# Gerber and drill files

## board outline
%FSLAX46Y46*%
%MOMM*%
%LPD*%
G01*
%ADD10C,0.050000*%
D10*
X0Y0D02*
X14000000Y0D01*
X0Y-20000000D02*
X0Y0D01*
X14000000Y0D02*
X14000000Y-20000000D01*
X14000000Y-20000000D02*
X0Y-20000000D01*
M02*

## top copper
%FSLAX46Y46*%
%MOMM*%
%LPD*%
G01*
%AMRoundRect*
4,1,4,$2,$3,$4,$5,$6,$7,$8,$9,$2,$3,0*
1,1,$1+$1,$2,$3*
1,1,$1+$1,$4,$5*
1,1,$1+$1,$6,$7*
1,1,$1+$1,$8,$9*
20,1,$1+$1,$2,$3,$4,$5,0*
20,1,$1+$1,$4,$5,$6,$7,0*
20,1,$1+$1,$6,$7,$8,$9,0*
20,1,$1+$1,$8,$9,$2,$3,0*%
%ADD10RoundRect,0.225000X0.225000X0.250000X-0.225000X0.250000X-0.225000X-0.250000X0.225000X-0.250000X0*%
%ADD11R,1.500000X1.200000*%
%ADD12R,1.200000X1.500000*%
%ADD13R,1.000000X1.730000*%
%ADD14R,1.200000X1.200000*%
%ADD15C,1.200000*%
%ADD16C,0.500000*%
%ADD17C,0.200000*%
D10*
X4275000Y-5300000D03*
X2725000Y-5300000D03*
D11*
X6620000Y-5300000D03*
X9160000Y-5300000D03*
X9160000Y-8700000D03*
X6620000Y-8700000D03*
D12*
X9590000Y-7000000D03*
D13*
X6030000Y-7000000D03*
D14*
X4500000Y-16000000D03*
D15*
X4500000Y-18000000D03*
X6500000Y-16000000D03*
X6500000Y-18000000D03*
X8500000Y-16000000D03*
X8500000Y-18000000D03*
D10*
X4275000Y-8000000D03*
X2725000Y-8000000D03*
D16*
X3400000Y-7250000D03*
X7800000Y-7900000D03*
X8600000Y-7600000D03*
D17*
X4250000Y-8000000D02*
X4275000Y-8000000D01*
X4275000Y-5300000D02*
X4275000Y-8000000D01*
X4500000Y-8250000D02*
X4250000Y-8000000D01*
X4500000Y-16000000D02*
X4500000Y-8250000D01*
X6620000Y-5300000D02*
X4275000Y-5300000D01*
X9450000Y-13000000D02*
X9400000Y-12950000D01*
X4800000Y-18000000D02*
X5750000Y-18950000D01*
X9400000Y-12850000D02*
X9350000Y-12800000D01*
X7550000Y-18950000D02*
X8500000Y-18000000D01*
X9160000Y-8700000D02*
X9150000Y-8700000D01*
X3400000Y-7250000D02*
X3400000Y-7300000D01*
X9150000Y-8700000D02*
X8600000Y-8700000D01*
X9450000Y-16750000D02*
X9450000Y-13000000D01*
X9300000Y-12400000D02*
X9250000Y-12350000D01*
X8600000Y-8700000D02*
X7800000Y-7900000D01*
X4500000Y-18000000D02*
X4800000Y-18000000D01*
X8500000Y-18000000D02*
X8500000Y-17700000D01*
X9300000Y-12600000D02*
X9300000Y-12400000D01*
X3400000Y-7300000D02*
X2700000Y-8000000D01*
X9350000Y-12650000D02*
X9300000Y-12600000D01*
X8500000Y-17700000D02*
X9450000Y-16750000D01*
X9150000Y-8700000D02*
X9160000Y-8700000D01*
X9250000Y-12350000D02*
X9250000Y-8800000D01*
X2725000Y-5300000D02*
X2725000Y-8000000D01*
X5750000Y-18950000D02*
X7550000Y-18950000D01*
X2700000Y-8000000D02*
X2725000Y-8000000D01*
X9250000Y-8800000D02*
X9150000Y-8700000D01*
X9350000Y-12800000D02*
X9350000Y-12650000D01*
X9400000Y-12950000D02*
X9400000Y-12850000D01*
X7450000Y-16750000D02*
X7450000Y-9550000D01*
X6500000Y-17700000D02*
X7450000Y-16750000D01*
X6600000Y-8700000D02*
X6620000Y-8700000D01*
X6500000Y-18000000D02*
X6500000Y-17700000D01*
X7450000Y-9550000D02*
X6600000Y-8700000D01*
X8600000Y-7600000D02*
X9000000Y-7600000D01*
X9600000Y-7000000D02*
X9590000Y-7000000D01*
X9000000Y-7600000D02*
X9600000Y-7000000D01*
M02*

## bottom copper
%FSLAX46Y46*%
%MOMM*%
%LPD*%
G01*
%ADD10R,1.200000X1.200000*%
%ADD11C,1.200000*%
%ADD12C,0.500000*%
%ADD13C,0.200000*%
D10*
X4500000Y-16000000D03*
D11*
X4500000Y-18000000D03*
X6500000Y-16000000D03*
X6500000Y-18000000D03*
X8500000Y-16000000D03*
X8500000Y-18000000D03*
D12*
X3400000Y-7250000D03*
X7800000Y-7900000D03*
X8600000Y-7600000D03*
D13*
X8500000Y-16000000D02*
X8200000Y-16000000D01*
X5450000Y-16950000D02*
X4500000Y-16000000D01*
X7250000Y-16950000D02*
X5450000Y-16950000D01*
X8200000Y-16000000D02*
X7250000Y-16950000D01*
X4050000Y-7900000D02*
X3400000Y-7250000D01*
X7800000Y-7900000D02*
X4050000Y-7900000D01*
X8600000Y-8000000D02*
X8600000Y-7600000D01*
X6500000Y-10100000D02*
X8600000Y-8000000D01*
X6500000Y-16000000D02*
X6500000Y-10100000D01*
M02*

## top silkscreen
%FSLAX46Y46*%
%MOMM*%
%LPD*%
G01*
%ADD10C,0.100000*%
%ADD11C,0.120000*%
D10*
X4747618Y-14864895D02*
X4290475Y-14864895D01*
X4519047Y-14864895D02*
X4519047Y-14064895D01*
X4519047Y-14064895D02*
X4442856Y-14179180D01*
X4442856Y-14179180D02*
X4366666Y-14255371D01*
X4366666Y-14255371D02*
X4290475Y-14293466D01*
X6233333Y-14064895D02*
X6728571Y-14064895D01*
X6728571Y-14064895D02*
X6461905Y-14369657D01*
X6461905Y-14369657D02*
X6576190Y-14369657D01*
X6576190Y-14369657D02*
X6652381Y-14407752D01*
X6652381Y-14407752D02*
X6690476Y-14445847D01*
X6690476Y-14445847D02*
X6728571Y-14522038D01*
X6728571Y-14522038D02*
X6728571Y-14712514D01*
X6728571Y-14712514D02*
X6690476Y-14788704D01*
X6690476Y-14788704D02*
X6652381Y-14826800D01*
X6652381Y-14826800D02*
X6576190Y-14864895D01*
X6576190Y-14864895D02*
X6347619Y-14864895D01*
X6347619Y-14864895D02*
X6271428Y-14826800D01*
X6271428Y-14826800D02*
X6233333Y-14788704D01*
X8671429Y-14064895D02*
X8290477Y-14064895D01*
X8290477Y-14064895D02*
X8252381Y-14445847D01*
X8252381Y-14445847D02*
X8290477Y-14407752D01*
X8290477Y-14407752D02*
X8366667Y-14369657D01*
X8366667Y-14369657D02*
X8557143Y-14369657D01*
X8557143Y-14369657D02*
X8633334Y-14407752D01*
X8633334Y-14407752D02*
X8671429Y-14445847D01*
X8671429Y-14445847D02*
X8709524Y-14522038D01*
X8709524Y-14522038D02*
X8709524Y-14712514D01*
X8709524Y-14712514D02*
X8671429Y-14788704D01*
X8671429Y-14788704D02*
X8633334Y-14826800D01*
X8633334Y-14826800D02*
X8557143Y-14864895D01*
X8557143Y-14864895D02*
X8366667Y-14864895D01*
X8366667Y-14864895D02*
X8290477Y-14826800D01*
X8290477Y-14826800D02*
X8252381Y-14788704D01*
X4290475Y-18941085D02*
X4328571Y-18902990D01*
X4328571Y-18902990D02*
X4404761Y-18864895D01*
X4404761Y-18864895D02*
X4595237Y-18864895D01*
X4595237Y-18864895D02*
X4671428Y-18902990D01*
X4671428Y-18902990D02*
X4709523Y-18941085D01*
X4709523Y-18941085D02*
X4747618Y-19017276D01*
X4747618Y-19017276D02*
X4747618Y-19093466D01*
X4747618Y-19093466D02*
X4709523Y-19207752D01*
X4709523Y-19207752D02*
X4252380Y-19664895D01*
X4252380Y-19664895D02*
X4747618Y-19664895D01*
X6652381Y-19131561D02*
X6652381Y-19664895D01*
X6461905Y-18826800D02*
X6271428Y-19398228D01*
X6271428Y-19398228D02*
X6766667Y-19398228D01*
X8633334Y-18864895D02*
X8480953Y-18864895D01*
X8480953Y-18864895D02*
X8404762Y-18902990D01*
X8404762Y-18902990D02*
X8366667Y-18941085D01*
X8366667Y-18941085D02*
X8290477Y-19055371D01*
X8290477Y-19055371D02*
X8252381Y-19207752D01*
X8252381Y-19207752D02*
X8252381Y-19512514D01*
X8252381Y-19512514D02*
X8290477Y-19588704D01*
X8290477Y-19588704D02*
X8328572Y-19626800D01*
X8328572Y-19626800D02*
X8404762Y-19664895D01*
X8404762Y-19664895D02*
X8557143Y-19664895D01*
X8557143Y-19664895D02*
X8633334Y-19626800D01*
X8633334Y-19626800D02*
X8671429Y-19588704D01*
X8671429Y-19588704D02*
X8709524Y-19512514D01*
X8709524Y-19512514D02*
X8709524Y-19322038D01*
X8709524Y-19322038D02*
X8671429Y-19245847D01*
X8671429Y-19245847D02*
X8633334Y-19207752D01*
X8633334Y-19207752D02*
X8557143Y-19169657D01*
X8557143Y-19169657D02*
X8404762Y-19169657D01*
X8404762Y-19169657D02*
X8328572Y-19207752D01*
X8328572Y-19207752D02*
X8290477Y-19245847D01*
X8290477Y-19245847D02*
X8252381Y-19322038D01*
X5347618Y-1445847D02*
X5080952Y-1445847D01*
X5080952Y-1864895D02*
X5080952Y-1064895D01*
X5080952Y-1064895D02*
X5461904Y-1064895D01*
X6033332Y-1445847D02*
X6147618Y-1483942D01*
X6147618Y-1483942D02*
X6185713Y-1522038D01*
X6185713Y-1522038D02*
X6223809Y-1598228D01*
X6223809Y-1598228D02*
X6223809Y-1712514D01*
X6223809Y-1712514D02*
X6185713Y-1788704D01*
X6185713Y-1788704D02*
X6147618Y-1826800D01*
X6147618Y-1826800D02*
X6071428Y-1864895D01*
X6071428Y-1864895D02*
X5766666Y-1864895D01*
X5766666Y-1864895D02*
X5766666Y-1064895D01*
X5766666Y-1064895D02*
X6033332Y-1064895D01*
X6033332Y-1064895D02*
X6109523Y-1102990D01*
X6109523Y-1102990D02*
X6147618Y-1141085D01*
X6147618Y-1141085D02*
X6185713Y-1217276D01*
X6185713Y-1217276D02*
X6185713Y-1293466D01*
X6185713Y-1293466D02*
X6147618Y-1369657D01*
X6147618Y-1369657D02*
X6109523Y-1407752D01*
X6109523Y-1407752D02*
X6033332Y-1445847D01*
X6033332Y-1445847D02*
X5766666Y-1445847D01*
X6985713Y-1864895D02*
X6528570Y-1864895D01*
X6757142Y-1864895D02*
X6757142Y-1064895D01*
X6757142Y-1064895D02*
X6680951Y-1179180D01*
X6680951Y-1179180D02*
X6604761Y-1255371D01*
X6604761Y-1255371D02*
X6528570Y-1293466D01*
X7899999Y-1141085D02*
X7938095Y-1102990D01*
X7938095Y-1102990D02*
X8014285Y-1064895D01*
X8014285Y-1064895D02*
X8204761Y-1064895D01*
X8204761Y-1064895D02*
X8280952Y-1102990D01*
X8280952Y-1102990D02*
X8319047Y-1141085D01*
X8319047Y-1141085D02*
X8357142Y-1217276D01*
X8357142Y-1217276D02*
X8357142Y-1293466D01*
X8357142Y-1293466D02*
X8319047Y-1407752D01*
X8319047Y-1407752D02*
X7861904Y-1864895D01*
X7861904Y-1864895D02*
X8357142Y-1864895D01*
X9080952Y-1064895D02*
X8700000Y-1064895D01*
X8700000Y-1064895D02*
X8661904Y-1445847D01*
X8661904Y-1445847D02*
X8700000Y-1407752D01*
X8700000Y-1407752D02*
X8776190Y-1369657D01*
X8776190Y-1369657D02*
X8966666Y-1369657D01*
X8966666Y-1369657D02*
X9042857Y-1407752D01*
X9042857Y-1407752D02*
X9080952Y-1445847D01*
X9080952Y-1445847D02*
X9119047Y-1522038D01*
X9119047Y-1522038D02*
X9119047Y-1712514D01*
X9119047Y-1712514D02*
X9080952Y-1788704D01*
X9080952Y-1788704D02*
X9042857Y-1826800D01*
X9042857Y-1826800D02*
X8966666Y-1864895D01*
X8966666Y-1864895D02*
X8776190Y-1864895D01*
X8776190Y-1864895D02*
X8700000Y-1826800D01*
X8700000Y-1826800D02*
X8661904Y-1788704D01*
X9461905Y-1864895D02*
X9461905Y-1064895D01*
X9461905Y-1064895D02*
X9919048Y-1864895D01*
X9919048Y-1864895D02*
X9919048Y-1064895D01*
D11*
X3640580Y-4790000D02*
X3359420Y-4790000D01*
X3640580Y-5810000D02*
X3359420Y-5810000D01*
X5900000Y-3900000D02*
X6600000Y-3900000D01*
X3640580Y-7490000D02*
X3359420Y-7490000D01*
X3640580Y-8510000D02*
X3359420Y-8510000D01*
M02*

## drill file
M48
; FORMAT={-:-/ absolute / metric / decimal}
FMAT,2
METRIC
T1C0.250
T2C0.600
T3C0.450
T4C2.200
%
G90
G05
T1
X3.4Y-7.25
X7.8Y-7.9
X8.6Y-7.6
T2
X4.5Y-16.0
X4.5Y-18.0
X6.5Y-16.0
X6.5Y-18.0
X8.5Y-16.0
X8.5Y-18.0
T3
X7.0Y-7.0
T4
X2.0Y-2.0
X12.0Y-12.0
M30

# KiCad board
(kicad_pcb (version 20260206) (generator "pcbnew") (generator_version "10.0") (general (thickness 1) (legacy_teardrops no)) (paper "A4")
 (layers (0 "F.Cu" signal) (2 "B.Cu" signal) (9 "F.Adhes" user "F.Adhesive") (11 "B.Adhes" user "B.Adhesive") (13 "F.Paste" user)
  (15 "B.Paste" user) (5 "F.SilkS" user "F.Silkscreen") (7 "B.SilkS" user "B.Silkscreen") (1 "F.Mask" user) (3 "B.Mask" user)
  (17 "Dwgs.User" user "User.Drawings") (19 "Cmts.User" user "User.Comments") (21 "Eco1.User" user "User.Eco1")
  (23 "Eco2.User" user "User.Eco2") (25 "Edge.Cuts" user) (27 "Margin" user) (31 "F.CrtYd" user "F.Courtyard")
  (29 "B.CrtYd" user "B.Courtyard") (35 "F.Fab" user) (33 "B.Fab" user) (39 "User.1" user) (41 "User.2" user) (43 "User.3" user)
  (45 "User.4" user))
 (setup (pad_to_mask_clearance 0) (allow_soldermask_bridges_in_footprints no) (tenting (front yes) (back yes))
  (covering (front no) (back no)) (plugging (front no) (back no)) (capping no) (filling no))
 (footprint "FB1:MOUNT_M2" (layer "F.Cu") (at 2 2)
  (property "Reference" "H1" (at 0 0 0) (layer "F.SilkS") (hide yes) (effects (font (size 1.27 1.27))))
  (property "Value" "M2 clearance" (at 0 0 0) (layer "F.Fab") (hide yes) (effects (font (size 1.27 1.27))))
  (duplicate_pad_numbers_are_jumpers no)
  (pad "" np_thru_hole circle (at 0 0) (size 2.2 2.2) (drill 2.2) (layers "*.Cu")))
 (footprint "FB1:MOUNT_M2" (layer "F.Cu") (at 12 12)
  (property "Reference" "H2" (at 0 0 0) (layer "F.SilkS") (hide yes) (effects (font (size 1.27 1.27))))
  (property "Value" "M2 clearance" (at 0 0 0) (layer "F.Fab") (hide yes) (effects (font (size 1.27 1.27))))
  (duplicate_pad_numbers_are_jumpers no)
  (pad "" np_thru_hole circle (at 0 0) (size 2.2 2.2) (drill 2.2) (layers "*.Cu")))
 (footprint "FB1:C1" (layer "F.Cu") (at 3.5 5.3 180)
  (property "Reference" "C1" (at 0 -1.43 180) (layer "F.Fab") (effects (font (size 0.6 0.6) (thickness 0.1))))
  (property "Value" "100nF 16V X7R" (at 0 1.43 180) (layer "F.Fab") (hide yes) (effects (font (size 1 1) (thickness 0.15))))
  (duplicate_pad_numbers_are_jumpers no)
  (fp_line (start -0.14058 0.51) (end 0.14058 0.51) (stroke (width 0.12) (type solid)) (layer "F.SilkS"))
  (fp_line (start -0.14058 -0.51) (end 0.14058 -0.51) (stroke (width 0.12) (type solid)) (layer "F.SilkS"))
  (pad "1" smd roundrect (at -0.775 0 180) (size 0.9 0.95) (layers "F.Cu" "F.Mask" "F.Paste") (roundrect_rratio 0.25) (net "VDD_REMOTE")
   (solder_mask_margin 0.025))
  (pad "2" smd roundrect (at 0.775 0 180) (size 0.9 0.95) (layers "F.Cu" "F.Mask" "F.Paste") (roundrect_rratio 0.25) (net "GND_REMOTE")
   (solder_mask_margin 0.025)))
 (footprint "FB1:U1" (layer "F.Cu") (at 7 7)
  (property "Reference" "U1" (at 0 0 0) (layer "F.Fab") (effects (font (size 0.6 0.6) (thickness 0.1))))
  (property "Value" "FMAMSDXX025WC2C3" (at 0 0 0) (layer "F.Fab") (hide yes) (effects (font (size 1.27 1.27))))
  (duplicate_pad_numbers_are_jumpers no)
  (fp_line (start -1.1 -3.1) (end -0.4 -3.1) (stroke (width 0.12) (type default)) (layer "F.SilkS"))
  (pad "" np_thru_hole circle (at 0 0) (size 0.45 0.45) (drill 0.45) (layers "*.Cu") (solder_mask_margin 0.025))
  (pad "1" smd rect (at -0.38 -1.7) (size 1.5 1.2) (layers "F.Cu" "F.Mask" "F.Paste") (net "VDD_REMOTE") (solder_mask_margin 0.025)
   (thermal_bridge_angle 45))
  (pad "2" smd rect (at 2.16 -1.7) (size 1.5 1.2) (layers "F.Cu" "F.Mask" "F.Paste") (solder_mask_margin 0.025) (thermal_bridge_angle 45))
  (pad "3" smd rect (at 2.16 1.7) (size 1.5 1.2) (layers "F.Cu" "F.Mask" "F.Paste") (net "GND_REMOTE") (solder_mask_margin 0.025)
   (thermal_bridge_angle 45))
  (pad "4" smd rect (at -0.38 1.7) (size 1.5 1.2) (layers "F.Cu" "F.Mask" "F.Paste") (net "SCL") (solder_mask_margin 0.025)
   (thermal_bridge_angle 45))
  (pad "5" smd rect (at 2.59 0) (size 1.2 1.5) (layers "F.Cu" "F.Mask" "F.Paste") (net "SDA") (solder_mask_margin 0.025)
   (thermal_bridge_angle 45))
  (pad "6" smd rect (at -0.97 0) (size 1 1.73) (layers "F.Cu" "F.Mask" "F.Paste") (solder_mask_margin 0.025) (thermal_bridge_angle 45)))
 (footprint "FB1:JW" (layer "F.Cu") (at 0 0)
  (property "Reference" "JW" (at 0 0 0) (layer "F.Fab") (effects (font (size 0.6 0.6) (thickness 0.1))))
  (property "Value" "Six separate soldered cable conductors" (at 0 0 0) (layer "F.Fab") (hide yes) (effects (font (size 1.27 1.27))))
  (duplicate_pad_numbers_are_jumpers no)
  (pad "1" thru_hole rect (at 4.5 16) (size 1.2 1.2) (drill 0.6) (layers "*.Cu") (remove_unused_layers no) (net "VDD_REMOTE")
   (solder_mask_margin 0.025) (thermal_bridge_angle 45))
  (pad "2" thru_hole circle (at 4.5 18) (size 1.2 1.2) (drill 0.6) (layers "*.Cu") (remove_unused_layers no) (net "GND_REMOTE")
   (solder_mask_margin 0.025))
  (pad "3" thru_hole circle (at 6.5 16) (size 1.2 1.2) (drill 0.6) (layers "*.Cu") (remove_unused_layers no) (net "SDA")
   (solder_mask_margin 0.025))
  (pad "4" thru_hole circle (at 6.5 18) (size 1.2 1.2) (drill 0.6) (layers "*.Cu") (remove_unused_layers no) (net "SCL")
   (solder_mask_margin 0.025))
  (pad "5" thru_hole circle (at 8.5 16) (size 1.2 1.2) (drill 0.6) (layers "*.Cu") (remove_unused_layers no) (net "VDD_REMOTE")
   (solder_mask_margin 0.025))
  (pad "6" thru_hole circle (at 8.5 18) (size 1.2 1.2) (drill 0.6) (layers "*.Cu") (remove_unused_layers no) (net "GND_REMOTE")
   (solder_mask_margin 0.025)))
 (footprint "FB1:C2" (layer "F.Cu") (at 3.5 8 180)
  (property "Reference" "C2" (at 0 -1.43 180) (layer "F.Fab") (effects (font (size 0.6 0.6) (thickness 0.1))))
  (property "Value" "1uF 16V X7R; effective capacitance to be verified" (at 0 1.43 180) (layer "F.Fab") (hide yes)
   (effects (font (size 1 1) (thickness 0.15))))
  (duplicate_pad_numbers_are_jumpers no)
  (fp_line (start -0.14058 0.51) (end 0.14058 0.51) (stroke (width 0.12) (type solid)) (layer "F.SilkS"))
  (fp_line (start -0.14058 -0.51) (end 0.14058 -0.51) (stroke (width 0.12) (type solid)) (layer "F.SilkS"))
  (pad "1" smd roundrect (at -0.775 0 180) (size 0.9 0.95) (layers "F.Cu" "F.Mask" "F.Paste") (roundrect_rratio 0.25) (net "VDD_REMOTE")
   (solder_mask_margin 0.025))
  (pad "2" smd roundrect (at 0.775 0 180) (size 0.9 0.95) (layers "F.Cu" "F.Mask" "F.Paste") (roundrect_rratio 0.25) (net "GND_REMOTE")
   (solder_mask_margin 0.025)))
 (gr_line (start 0 0) (end 14 0) (stroke (width 0.05) (type default)) (layer "Edge.Cuts"))
 (gr_line (start 0 20) (end 0 0) (stroke (width 0.05) (type default)) (layer "Edge.Cuts"))
 (gr_line (start 14 0) (end 14 20) (stroke (width 0.05) (type default)) (layer "Edge.Cuts"))
 (gr_line (start 14 20) (end 0 20) (stroke (width 0.05) (type default)) (layer "Edge.Cuts"))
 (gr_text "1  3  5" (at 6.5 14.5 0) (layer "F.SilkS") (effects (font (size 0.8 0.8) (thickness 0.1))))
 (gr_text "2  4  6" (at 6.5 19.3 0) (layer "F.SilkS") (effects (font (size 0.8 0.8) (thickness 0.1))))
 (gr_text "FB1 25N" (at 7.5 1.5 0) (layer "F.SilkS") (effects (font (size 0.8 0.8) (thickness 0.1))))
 (segment (start 4.25 8) (end 4.275 8) (width 0.2) (layer "F.Cu") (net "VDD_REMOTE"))
 (segment (start 4.275 5.3) (end 4.275 8) (width 0.2) (layer "F.Cu") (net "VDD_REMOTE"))
 (segment (start 4.5 8.25) (end 4.25 8) (width 0.2) (layer "F.Cu") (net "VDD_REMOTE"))
 (segment (start 4.5 16) (end 4.5 8.25) (width 0.2) (layer "F.Cu") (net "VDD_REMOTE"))
 (segment (start 6.62 5.3) (end 4.275 5.3) (width 0.2) (layer "F.Cu") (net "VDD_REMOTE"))
 (segment (start 8.5 16) (end 8.2 16) (width 0.2) (layer "B.Cu") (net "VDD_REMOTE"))
 (segment (start 5.45 16.95) (end 4.5 16) (width 0.2) (layer "B.Cu") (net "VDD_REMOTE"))
 (segment (start 7.25 16.95) (end 5.45 16.95) (width 0.2) (layer "B.Cu") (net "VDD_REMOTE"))
 (segment (start 8.2 16) (end 7.25 16.95) (width 0.2) (layer "B.Cu") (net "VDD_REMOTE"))
 (segment (start 9.45 13) (end 9.4 12.95) (width 0.2) (layer "F.Cu") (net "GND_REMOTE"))
 (segment (start 4.8 18) (end 5.75 18.95) (width 0.2) (layer "F.Cu") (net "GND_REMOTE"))
 (segment (start 9.4 12.85) (end 9.35 12.8) (width 0.2) (layer "F.Cu") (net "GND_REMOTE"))
 (segment (start 7.55 18.95) (end 8.5 18) (width 0.2) (layer "F.Cu") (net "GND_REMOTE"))
 (segment (start 9.16 8.7) (end 9.15 8.7) (width 0.2) (layer "F.Cu") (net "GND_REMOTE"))
 (segment (start 3.4 7.25) (end 3.4 7.3) (width 0.2) (layer "F.Cu") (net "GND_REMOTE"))
 (segment (start 9.15 8.7) (end 8.6 8.7) (width 0.2) (layer "F.Cu") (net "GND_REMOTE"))
 (segment (start 9.45 16.75) (end 9.45 13) (width 0.2) (layer "F.Cu") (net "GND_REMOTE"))
 (segment (start 9.3 12.4) (end 9.25 12.35) (width 0.2) (layer "F.Cu") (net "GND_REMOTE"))
 (segment (start 8.6 8.7) (end 7.8 7.9) (width 0.2) (layer "F.Cu") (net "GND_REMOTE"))
 (segment (start 4.5 18) (end 4.8 18) (width 0.2) (layer "F.Cu") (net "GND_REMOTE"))
 (segment (start 8.5 18) (end 8.5 17.7) (width 0.2) (layer "F.Cu") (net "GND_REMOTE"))
 (segment (start 9.3 12.6) (end 9.3 12.4) (width 0.2) (layer "F.Cu") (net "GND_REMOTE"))
 (segment (start 3.4 7.3) (end 2.7 8) (width 0.2) (layer "F.Cu") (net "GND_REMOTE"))
 (segment (start 9.35 12.65) (end 9.3 12.6) (width 0.2) (layer "F.Cu") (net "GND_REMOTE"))
 (segment (start 8.5 17.7) (end 9.45 16.75) (width 0.2) (layer "F.Cu") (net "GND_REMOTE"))
 (segment (start 9.15 8.7) (end 9.16 8.7) (width 0.2) (layer "F.Cu") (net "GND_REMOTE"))
 (segment (start 9.25 12.35) (end 9.25 8.8) (width 0.2) (layer "F.Cu") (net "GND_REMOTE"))
 (segment (start 2.725 5.3) (end 2.725 8) (width 0.2) (layer "F.Cu") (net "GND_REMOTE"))
 (segment (start 5.75 18.95) (end 7.55 18.95) (width 0.2) (layer "F.Cu") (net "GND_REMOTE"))
 (segment (start 2.7 8) (end 2.725 8) (width 0.2) (layer "F.Cu") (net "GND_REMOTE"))
 (segment (start 9.25 8.8) (end 9.15 8.7) (width 0.2) (layer "F.Cu") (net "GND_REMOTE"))
 (segment (start 9.35 12.8) (end 9.35 12.65) (width 0.2) (layer "F.Cu") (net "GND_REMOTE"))
 (segment (start 9.4 12.95) (end 9.4 12.85) (width 0.2) (layer "F.Cu") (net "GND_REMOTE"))
 (via (at 3.4 7.25) (size 0.5) (drill 0.25) (layers "F.Cu" "B.Cu") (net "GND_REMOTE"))
 (via (at 7.8 7.9) (size 0.5) (drill 0.25) (layers "F.Cu" "B.Cu") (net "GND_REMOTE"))
 (segment (start 4.05 7.9) (end 3.4 7.25) (width 0.2) (layer "B.Cu") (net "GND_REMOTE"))
 (segment (start 7.8 7.9) (end 4.05 7.9) (width 0.2) (layer "B.Cu") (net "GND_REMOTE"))
 (segment (start 7.45 16.75) (end 7.45 9.55) (width 0.2) (layer "F.Cu") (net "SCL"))
 (segment (start 6.5 17.7) (end 7.45 16.75) (width 0.2) (layer "F.Cu") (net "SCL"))
 (segment (start 6.6 8.7) (end 6.62 8.7) (width 0.2) (layer "F.Cu") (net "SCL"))
 (segment (start 6.5 18) (end 6.5 17.7) (width 0.2) (layer "F.Cu") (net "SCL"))
 (segment (start 7.45 9.55) (end 6.6 8.7) (width 0.2) (layer "F.Cu") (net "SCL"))
 (segment (start 8.6 7.6) (end 9 7.6) (width 0.2) (layer "F.Cu") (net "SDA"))
 (segment (start 9.6 7) (end 9.59 7) (width 0.2) (layer "F.Cu") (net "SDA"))
 (segment (start 9 7.6) (end 9.6 7) (width 0.2) (layer "F.Cu") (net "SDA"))
 (via (at 8.6 7.6) (size 0.5) (drill 0.25) (layers "F.Cu" "B.Cu") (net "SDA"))
 (segment (start 8.6 8) (end 8.6 7.6) (width 0.2) (layer "B.Cu") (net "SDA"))
 (segment (start 6.5 10.1) (end 8.6 8) (width 0.2) (layer "B.Cu") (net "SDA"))
 (segment (start 6.5 16) (end 6.5 10.1) (width 0.2) (layer "B.Cu") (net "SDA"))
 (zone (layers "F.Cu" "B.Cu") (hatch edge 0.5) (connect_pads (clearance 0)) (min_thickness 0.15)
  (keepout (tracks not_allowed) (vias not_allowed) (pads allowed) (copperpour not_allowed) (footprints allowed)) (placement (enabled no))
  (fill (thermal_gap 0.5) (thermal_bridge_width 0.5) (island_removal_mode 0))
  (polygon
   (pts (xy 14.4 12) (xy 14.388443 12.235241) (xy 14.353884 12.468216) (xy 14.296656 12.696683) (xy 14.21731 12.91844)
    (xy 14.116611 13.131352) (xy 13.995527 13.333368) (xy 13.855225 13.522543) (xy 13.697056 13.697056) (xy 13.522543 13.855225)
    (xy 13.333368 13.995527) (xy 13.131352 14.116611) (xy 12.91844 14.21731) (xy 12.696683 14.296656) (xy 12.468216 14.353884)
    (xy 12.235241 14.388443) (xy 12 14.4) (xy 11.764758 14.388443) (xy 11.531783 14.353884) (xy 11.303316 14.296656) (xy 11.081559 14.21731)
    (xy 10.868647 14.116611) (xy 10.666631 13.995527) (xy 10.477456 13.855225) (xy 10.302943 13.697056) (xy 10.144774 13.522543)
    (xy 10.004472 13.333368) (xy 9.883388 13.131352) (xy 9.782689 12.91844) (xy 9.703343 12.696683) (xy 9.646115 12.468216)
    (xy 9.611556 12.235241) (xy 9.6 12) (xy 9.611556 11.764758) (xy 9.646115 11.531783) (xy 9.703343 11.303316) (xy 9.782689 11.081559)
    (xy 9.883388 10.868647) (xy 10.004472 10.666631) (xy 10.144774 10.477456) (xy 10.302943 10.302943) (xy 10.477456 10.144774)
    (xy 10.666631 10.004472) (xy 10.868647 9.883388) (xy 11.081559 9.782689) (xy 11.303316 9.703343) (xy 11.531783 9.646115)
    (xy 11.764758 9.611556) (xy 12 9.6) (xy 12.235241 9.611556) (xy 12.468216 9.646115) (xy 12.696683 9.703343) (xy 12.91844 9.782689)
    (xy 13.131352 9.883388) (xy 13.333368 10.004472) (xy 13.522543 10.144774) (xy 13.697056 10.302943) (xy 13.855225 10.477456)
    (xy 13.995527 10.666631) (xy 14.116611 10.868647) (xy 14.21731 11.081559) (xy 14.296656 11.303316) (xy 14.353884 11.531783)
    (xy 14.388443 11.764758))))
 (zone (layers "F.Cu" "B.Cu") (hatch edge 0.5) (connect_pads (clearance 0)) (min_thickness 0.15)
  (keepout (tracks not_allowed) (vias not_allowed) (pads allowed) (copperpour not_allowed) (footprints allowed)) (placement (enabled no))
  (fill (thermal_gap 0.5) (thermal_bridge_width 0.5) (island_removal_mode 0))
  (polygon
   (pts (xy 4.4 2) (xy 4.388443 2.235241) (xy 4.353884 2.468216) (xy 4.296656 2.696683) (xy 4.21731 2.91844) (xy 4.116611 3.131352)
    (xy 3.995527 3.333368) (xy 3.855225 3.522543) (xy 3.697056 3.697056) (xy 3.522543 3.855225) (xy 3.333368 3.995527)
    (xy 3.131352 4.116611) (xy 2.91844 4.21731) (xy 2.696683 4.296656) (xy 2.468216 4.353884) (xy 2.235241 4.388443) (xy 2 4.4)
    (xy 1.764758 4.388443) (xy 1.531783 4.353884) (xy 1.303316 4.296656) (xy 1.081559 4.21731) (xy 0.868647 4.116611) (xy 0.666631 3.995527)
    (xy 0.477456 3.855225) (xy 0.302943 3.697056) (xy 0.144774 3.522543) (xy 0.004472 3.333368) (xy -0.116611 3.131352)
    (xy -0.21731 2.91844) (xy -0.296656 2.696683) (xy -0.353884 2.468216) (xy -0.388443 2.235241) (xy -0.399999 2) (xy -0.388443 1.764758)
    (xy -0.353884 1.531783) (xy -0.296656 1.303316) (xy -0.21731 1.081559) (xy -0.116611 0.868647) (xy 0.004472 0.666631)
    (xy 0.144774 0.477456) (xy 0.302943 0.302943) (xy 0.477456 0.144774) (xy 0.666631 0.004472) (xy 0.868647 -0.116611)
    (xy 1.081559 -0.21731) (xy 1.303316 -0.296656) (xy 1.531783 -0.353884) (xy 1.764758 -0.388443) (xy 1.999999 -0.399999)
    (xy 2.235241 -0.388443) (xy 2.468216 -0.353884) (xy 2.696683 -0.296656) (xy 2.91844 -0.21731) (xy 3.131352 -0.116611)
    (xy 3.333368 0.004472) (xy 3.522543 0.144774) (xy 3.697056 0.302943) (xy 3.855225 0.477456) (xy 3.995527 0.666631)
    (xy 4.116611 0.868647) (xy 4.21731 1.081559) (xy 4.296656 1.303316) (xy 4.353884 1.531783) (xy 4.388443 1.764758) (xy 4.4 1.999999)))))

